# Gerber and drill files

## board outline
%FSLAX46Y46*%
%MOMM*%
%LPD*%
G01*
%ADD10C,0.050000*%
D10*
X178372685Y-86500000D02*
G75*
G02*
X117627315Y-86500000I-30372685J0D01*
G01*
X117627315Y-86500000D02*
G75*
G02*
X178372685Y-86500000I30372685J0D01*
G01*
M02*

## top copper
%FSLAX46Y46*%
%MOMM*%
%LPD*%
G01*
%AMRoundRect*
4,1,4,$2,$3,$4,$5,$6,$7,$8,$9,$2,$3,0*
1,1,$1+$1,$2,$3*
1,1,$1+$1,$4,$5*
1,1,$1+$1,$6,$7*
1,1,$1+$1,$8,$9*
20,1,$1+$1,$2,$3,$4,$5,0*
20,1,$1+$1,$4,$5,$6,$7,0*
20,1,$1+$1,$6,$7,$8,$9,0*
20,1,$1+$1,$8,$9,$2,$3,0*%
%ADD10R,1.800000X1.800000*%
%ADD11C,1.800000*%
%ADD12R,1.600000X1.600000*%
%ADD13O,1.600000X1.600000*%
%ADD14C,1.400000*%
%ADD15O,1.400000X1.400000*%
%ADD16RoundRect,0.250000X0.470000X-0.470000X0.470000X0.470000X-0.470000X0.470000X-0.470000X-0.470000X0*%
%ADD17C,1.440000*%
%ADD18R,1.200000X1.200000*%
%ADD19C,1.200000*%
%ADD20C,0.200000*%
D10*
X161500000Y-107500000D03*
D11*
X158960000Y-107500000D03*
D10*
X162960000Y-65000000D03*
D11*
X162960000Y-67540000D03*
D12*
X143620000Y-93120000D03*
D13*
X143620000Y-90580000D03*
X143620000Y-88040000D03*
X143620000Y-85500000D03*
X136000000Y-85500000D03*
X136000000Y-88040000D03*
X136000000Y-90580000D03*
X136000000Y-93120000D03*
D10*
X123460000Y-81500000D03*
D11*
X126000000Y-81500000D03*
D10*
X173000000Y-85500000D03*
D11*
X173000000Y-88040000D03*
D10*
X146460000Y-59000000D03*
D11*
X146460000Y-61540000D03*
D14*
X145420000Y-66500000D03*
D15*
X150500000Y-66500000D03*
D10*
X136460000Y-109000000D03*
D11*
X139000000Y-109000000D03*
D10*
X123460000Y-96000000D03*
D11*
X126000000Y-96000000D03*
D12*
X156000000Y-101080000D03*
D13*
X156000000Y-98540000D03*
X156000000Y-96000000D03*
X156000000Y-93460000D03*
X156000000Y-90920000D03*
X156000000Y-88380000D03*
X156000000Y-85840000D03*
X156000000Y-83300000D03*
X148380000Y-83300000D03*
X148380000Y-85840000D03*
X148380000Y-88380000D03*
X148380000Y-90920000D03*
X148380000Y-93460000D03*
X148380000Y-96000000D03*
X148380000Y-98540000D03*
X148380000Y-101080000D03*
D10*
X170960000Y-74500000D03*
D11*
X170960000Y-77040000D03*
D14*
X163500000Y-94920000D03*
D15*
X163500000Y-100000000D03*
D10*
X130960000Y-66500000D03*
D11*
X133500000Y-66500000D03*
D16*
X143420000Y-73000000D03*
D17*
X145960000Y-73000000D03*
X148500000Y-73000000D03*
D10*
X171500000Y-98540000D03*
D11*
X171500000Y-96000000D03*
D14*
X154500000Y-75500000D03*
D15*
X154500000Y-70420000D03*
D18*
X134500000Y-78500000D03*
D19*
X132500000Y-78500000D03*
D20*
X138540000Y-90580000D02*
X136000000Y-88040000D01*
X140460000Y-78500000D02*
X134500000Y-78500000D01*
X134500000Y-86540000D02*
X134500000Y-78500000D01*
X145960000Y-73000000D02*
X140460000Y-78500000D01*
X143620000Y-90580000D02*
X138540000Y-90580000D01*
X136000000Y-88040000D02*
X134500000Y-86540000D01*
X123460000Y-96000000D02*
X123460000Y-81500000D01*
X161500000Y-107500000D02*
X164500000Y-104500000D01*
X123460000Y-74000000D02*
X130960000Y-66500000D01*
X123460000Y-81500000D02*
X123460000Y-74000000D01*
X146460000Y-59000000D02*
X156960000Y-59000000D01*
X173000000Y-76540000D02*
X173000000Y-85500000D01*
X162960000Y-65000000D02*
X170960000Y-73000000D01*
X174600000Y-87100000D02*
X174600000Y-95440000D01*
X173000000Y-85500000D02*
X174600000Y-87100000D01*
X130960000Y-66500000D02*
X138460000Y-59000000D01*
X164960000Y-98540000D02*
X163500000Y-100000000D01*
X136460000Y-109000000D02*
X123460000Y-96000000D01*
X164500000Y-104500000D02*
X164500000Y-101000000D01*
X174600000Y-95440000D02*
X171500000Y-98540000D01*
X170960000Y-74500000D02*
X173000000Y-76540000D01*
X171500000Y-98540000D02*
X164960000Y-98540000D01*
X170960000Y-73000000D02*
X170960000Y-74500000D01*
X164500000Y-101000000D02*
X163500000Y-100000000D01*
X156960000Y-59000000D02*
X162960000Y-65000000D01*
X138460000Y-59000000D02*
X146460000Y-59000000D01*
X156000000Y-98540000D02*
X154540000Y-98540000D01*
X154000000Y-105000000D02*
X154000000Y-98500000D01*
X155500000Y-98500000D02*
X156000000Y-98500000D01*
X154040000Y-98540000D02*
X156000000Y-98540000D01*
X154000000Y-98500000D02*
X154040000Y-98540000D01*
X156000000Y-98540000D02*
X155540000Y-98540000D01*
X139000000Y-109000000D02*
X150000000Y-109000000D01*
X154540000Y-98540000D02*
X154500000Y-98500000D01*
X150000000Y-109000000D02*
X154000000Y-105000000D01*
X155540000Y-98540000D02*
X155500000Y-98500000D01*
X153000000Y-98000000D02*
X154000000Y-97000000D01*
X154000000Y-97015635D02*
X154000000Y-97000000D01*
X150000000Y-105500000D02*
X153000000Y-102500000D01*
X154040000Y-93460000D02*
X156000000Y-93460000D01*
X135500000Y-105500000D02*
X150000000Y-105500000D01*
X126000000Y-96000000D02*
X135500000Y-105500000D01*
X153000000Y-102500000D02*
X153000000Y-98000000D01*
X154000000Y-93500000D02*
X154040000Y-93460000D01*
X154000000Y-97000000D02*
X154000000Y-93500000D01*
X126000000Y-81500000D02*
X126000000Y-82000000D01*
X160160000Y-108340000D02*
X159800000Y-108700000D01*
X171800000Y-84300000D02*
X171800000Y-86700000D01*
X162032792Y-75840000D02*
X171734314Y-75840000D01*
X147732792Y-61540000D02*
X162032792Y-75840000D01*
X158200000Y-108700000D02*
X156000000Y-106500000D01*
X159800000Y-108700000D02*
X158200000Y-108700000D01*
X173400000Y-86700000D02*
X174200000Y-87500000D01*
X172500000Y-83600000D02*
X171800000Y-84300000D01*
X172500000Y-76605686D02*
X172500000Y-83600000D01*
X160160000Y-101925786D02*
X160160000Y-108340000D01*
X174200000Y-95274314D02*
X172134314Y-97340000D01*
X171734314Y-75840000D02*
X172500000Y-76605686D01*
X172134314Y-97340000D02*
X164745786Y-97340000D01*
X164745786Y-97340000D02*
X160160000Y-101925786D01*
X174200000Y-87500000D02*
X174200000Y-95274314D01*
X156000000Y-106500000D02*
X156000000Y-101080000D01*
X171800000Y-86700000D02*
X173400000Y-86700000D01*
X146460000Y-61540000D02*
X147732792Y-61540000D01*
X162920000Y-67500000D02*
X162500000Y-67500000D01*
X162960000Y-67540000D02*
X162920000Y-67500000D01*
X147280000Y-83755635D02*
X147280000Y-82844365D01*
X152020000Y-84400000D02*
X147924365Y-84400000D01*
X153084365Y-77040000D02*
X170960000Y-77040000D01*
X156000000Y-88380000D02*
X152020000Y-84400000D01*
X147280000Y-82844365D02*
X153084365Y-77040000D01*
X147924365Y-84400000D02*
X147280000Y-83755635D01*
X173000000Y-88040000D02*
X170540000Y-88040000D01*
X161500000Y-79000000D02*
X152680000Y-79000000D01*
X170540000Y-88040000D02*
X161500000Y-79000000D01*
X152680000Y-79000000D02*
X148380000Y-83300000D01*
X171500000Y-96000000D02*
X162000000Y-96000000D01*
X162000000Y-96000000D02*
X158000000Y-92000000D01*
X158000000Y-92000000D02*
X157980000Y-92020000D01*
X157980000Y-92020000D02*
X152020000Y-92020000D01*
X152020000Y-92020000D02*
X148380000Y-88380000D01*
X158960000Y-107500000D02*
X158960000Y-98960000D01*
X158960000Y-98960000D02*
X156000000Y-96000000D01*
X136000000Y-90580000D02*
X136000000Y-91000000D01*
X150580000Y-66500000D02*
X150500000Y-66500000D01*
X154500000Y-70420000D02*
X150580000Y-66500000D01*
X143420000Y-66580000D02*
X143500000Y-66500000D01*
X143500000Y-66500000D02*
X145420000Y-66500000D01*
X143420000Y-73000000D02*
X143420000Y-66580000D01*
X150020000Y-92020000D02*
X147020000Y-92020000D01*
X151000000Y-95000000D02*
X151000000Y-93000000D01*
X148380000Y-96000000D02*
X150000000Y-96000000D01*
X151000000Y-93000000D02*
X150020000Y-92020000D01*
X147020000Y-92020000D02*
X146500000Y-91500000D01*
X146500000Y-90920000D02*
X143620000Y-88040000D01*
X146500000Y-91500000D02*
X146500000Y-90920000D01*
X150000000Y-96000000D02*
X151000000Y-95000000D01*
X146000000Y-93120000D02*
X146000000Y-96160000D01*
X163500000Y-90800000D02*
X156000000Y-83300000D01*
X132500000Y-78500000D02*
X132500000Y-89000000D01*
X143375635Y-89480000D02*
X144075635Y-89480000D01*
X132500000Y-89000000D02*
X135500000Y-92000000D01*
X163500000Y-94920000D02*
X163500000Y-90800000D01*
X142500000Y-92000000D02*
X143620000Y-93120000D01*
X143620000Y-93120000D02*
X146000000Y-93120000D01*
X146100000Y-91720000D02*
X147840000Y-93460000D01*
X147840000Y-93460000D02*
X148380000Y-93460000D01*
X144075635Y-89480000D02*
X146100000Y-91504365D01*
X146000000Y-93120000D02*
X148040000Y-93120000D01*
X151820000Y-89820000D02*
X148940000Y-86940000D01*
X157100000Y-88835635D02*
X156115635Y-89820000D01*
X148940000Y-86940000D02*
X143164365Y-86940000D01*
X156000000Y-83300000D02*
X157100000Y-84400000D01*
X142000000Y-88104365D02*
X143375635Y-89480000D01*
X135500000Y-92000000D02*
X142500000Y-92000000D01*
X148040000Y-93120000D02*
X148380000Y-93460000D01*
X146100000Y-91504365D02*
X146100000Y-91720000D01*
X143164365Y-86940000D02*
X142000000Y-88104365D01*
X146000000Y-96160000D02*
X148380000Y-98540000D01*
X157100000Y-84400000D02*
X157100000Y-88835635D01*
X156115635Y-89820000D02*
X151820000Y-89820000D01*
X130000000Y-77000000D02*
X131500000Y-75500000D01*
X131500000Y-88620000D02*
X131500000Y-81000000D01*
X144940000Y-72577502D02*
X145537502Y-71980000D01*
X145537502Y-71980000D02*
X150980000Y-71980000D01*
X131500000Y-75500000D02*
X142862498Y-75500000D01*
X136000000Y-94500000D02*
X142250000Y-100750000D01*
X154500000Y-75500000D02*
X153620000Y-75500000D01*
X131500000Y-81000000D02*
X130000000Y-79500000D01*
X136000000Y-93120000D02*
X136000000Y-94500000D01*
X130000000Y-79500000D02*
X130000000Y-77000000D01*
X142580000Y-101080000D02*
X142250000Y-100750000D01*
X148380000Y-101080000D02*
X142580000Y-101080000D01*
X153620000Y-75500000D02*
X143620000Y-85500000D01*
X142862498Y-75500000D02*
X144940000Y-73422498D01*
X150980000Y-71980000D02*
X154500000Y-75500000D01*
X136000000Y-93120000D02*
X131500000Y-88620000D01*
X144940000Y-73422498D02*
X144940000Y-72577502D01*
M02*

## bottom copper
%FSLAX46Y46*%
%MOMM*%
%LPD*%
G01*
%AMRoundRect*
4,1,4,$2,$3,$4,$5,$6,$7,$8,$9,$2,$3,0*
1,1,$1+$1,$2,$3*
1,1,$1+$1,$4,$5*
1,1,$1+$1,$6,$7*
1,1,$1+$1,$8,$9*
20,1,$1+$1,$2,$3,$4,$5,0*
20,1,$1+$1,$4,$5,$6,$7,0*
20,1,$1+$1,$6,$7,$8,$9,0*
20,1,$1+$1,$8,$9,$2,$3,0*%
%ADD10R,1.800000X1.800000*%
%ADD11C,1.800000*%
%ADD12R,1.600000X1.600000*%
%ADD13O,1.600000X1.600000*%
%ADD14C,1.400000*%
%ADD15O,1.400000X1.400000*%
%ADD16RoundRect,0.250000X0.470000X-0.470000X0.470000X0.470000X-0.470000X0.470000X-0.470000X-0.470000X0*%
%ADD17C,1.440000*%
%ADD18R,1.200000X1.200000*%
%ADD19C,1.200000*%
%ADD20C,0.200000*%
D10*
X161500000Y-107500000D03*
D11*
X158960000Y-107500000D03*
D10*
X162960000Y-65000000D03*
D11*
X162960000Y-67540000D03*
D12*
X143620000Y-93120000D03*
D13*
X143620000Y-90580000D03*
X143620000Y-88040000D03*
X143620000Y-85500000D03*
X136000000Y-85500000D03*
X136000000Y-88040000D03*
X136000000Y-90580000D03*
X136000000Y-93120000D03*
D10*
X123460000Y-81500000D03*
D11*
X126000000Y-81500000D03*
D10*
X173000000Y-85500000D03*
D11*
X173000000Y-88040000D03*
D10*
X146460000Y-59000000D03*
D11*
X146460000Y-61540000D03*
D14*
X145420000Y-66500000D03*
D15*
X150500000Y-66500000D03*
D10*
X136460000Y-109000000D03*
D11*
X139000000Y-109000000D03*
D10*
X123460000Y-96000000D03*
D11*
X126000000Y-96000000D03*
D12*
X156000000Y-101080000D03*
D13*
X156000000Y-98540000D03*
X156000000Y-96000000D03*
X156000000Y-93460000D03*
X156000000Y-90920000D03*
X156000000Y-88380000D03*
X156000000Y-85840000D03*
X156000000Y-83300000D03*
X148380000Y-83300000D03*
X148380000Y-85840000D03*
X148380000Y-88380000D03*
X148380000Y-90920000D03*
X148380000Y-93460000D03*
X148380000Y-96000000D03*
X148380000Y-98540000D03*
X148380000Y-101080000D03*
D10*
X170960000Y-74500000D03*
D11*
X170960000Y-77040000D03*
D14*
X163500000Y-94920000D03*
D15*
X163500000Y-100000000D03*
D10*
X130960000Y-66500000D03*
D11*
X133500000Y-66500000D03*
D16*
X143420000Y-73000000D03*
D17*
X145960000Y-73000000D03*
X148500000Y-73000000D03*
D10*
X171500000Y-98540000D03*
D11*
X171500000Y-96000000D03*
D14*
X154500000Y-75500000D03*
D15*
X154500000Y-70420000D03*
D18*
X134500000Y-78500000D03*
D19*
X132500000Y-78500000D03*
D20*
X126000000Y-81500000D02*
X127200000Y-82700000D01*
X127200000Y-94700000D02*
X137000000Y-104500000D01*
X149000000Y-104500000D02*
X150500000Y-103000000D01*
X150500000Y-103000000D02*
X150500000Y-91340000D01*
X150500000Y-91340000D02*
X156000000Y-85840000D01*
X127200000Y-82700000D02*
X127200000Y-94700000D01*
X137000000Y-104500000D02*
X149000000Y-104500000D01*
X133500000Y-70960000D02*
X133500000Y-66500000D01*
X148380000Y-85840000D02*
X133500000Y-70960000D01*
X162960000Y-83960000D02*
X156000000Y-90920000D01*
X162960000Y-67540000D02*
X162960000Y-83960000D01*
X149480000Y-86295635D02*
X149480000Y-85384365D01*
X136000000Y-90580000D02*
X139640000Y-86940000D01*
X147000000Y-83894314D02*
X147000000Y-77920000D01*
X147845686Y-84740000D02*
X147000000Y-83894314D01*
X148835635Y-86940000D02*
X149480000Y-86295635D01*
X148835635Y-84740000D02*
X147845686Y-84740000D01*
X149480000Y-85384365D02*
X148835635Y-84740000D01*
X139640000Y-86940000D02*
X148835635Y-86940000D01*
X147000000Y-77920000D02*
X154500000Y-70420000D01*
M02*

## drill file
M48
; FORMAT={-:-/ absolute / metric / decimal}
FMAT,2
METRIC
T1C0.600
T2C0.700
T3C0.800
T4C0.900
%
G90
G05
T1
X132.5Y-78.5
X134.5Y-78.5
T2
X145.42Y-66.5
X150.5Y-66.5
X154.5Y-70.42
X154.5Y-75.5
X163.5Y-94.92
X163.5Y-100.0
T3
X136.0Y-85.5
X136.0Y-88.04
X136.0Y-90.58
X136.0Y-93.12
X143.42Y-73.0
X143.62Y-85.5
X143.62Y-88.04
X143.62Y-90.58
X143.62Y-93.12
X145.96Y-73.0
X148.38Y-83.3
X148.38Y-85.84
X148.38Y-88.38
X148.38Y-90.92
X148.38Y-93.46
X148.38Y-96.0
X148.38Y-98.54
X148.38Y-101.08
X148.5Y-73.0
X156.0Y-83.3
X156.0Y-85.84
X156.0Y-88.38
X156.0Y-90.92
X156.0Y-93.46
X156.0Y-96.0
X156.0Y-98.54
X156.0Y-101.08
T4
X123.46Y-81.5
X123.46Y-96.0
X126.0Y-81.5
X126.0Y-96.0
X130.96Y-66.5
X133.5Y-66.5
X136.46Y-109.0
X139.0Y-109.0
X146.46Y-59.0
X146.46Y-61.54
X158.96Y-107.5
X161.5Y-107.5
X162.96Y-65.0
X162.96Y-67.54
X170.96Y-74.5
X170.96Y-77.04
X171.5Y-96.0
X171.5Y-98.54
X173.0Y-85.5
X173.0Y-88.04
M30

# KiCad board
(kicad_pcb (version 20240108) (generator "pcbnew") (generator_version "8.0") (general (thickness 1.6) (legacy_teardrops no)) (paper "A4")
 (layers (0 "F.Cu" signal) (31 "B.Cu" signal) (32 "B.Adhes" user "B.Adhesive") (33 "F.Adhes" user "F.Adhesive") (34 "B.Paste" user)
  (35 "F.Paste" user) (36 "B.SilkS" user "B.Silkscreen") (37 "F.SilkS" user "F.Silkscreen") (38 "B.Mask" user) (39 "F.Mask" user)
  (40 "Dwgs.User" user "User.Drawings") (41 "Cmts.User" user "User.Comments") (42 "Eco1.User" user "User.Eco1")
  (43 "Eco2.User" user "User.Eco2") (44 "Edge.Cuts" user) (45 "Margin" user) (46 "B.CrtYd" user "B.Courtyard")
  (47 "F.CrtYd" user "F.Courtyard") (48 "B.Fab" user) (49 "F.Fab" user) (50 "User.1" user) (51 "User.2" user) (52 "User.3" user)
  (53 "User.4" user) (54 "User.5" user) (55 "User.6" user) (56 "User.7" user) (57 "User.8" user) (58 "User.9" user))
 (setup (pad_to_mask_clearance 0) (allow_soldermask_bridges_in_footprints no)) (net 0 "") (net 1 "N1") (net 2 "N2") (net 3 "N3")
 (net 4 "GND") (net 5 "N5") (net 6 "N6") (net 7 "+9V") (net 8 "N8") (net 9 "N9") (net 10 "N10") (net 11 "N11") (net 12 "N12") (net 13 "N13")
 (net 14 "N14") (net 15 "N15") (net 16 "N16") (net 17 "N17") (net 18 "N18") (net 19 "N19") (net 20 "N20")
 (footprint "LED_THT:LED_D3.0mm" (layer "F.Cu") (at 161.5 107.5 180)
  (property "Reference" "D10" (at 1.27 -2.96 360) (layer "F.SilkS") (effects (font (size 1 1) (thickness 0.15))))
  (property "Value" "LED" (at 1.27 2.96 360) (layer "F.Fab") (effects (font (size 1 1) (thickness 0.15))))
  (pad "1" thru_hole rect (at 0 0 180) (size 1.8 1.8) (drill 0.9) (layers "*.Cu" "*.Mask") (remove_unused_layers no) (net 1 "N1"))
  (pad "2" thru_hole circle (at 2.54 0 180) (size 1.8 1.8) (drill 0.9) (layers "*.Cu" "*.Mask") (remove_unused_layers no) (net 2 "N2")))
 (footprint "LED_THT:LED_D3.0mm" (layer "F.Cu") (at 162.96 65 -90)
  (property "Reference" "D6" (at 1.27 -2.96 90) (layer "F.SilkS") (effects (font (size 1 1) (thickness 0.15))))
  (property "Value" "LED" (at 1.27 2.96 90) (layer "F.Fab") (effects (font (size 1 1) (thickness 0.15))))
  (pad "1" thru_hole rect (at 0 0 270) (size 1.8 1.8) (drill 0.9) (layers "*.Cu" "*.Mask") (remove_unused_layers no) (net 1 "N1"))
  (pad "2" thru_hole circle (at 2.54 0 270) (size 1.8 1.8) (drill 0.9) (layers "*.Cu" "*.Mask") (remove_unused_layers no) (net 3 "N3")))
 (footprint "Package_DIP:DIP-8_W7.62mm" (layer "F.Cu") (at 143.62 93.12 180)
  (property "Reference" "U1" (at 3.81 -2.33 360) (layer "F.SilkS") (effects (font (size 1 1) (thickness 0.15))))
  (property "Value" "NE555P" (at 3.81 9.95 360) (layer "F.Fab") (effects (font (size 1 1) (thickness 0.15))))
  (pad "1" thru_hole rect (at 0 0 180) (size 1.6 1.6) (drill 0.8) (layers "*.Cu" "*.Mask") (remove_unused_layers no) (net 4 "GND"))
  (pad "2" thru_hole oval (at 0 2.54 180) (size 1.6 1.6) (drill 0.8) (layers "*.Cu" "*.Mask") (remove_unused_layers no) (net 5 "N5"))
  (pad "3" thru_hole oval (at 0 5.08 180) (size 1.6 1.6) (drill 0.8) (layers "*.Cu" "*.Mask") (remove_unused_layers no) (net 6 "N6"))
  (pad "4" thru_hole oval (at 0 7.62 180) (size 1.6 1.6) (drill 0.8) (layers "*.Cu" "*.Mask") (remove_unused_layers no) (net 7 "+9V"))
  (pad "5" thru_hole oval (at 7.62 7.62 180) (size 1.6 1.6) (drill 0.8) (layers "*.Cu" "*.Mask") (remove_unused_layers no) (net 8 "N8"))
  (pad "6" thru_hole oval (at 7.62 5.08 180) (size 1.6 1.6) (drill 0.8) (layers "*.Cu" "*.Mask") (remove_unused_layers no) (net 5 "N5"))
  (pad "7" thru_hole oval (at 7.62 2.54 180) (size 1.6 1.6) (drill 0.8) (layers "*.Cu" "*.Mask") (remove_unused_layers no) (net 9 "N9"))
  (pad "8" thru_hole oval (at 7.62 0 180) (size 1.6 1.6) (drill 0.8) (layers "*.Cu" "*.Mask") (remove_unused_layers no) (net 7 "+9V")))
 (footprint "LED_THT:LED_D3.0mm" (layer "F.Cu") (at 123.46 81.5)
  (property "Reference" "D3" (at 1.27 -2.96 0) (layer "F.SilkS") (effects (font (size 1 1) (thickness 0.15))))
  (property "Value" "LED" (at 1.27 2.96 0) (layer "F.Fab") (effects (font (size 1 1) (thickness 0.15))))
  (pad "1" thru_hole rect (at 0 0) (size 1.8 1.8) (drill 0.9) (layers "*.Cu" "*.Mask") (remove_unused_layers no) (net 1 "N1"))
  (pad "2" thru_hole circle (at 2.54 0) (size 1.8 1.8) (drill 0.9) (layers "*.Cu" "*.Mask") (remove_unused_layers no) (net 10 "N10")))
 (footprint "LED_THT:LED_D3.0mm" (layer "F.Cu") (at 173 85.5 -90)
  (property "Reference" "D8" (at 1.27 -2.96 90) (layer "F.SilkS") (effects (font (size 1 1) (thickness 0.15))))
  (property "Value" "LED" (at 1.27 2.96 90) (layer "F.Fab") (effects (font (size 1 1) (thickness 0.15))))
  (pad "1" thru_hole rect (at 0 0 270) (size 1.8 1.8) (drill 0.9) (layers "*.Cu" "*.Mask") (remove_unused_layers no) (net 1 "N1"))
  (pad "2" thru_hole circle (at 2.54 0 270) (size 1.8 1.8) (drill 0.9) (layers "*.Cu" "*.Mask") (remove_unused_layers no) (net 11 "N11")))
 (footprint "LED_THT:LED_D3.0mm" (layer "F.Cu") (at 146.46 59 -90)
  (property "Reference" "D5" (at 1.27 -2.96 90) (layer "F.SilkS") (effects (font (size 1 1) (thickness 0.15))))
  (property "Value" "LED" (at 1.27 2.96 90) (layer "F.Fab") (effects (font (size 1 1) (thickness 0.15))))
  (pad "1" thru_hole rect (at 0 0 270) (size 1.8 1.8) (drill 0.9) (layers "*.Cu" "*.Mask") (remove_unused_layers no) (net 1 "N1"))
  (pad "2" thru_hole circle (at 2.54 0 270) (size 1.8 1.8) (drill 0.9) (layers "*.Cu" "*.Mask") (remove_unused_layers no) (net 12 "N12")))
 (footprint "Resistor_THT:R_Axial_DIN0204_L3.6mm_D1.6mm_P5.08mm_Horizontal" (layer "F.Cu") (at 145.42 66.5)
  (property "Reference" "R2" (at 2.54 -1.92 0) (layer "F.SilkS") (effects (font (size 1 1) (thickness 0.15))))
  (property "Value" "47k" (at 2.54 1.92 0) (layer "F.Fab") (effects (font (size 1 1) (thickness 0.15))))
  (pad "1" thru_hole circle (at 0 0) (size 1.4 1.4) (drill 0.7) (layers "*.Cu" "*.Mask") (remove_unused_layers no) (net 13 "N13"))
  (pad "2" thru_hole oval (at 5.08 0) (size 1.4 1.4) (drill 0.7) (layers "*.Cu" "*.Mask") (remove_unused_layers no) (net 9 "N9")))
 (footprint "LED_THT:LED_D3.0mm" (layer "F.Cu") (at 136.46 109)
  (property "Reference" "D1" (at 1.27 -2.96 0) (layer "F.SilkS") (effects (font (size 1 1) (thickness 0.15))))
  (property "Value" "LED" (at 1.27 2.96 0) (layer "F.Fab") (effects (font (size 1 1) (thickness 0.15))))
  (pad "1" thru_hole rect (at 0 0) (size 1.8 1.8) (drill 0.9) (layers "*.Cu" "*.Mask") (remove_unused_layers no) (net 1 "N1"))
  (pad "2" thru_hole circle (at 2.54 0) (size 1.8 1.8) (drill 0.9) (layers "*.Cu" "*.Mask") (remove_unused_layers no) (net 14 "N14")))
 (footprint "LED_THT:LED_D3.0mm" (layer "F.Cu") (at 123.46 96)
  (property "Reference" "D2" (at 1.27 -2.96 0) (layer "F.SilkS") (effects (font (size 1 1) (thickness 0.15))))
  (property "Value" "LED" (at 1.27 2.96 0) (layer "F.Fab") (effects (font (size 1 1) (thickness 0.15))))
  (pad "1" thru_hole rect (at 0 0) (size 1.8 1.8) (drill 0.9) (layers "*.Cu" "*.Mask") (remove_unused_layers no) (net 1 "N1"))
  (pad "2" thru_hole circle (at 2.54 0) (size 1.8 1.8) (drill 0.9) (layers "*.Cu" "*.Mask") (remove_unused_layers no) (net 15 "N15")))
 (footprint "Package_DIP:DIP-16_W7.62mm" (layer "F.Cu") (at 156 101.08 180)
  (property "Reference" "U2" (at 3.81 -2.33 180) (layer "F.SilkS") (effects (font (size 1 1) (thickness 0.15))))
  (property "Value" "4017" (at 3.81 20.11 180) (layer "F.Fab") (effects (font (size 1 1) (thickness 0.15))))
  (pad "1" thru_hole rect (at 0 0 180) (size 1.6 1.6) (drill 0.8) (layers "*.Cu" "*.Mask") (remove_unused_layers no) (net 12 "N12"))
  (pad "2" thru_hole oval (at 0 2.54 180) (size 1.6 1.6) (drill 0.8) (layers "*.Cu" "*.Mask") (remove_unused_layers no) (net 14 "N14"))
  (pad "3" thru_hole oval (at 0 5.08 180) (size 1.6 1.6) (drill 0.8) (layers "*.Cu" "*.Mask") (remove_unused_layers no) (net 2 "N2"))
  (pad "4" thru_hole oval (at 0 7.62 180) (size 1.6 1.6) (drill 0.8) (layers "*.Cu" "*.Mask") (remove_unused_layers no) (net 15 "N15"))
  (pad "5" thru_hole oval (at 0 10.16 180) (size 1.6 1.6) (drill 0.8) (layers "*.Cu" "*.Mask") (remove_unused_layers no) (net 3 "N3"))
  (pad "6" thru_hole oval (at 0 12.7 180) (size 1.6 1.6) (drill 0.8) (layers "*.Cu" "*.Mask") (remove_unused_layers no) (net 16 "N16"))
  (pad "7" thru_hole oval (at 0 15.24 180) (size 1.6 1.6) (drill 0.8) (layers "*.Cu" "*.Mask") (remove_unused_layers no) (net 10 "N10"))
  (pad "8" thru_hole oval (at 0 17.78 180) (size 1.6 1.6) (drill 0.8) (layers "*.Cu" "*.Mask") (remove_unused_layers no) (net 4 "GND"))
  (pad "9" thru_hole oval (at 7.62 17.78 180) (size 1.6 1.6) (drill 0.8) (layers "*.Cu" "*.Mask") (remove_unused_layers no) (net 11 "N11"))
  (pad "10" thru_hole oval (at 7.62 15.24 180) (size 1.6 1.6) (drill 0.8) (layers "*.Cu" "*.Mask") (remove_unused_layers no) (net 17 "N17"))
  (pad "11" thru_hole oval (at 7.62 12.7 180) (size 1.6 1.6) (drill 0.8) (layers "*.Cu" "*.Mask") (remove_unused_layers no) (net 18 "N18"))
  (pad "12" thru_hole oval (at 7.62 10.16 180) (size 1.6 1.6) (drill 0.8) (layers "*.Cu" "*.Mask") (remove_unused_layers no) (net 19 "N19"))
  (pad "13" thru_hole oval (at 7.62 7.62 180) (size 1.6 1.6) (drill 0.8) (layers "*.Cu" "*.Mask") (remove_unused_layers no) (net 4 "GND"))
  (pad "14" thru_hole oval (at 7.62 5.08 180) (size 1.6 1.6) (drill 0.8) (layers "*.Cu" "*.Mask") (remove_unused_layers no) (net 6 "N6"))
  (pad "15" thru_hole oval (at 7.62 2.54 180) (size 1.6 1.6) (drill 0.8) (layers "*.Cu" "*.Mask") (remove_unused_layers no) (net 4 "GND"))
  (pad "16" thru_hole oval (at 7.62 0 180) (size 1.6 1.6) (drill 0.8) (layers "*.Cu" "*.Mask") (remove_unused_layers no) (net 7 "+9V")))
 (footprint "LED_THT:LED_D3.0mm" (layer "F.Cu") (at 170.96 74.5 -90)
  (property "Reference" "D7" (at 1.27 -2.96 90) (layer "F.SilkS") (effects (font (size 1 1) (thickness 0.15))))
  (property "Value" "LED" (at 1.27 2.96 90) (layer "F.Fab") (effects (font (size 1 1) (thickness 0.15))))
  (pad "1" thru_hole rect (at 0 0 270) (size 1.8 1.8) (drill 0.9) (layers "*.Cu" "*.Mask") (remove_unused_layers no) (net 1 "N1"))
  (pad "2" thru_hole circle (at 2.54 0 270) (size 1.8 1.8) (drill 0.9) (layers "*.Cu" "*.Mask") (remove_unused_layers no) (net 16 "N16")))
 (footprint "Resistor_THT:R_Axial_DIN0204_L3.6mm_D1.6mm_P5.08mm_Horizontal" (layer "F.Cu") (at 163.5 94.92 -90)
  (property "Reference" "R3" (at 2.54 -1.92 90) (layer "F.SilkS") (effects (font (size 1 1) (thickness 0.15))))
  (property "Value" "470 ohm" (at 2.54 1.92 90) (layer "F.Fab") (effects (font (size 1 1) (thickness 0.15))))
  (pad "1" thru_hole circle (at 0 0 270) (size 1.4 1.4) (drill 0.7) (layers "*.Cu" "*.Mask") (remove_unused_layers no) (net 4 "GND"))
  (pad "2" thru_hole oval (at 5.08 0 270) (size 1.4 1.4) (drill 0.7) (layers "*.Cu" "*.Mask") (remove_unused_layers no) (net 1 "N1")))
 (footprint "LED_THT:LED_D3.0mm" (layer "F.Cu") (at 130.96 66.5)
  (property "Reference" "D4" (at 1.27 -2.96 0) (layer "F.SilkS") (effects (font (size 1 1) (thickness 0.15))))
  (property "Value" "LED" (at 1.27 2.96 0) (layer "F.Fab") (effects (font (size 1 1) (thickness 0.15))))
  (pad "1" thru_hole rect (at 0 0) (size 1.8 1.8) (drill 0.9) (layers "*.Cu" "*.Mask") (remove_unused_layers no) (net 1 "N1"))
  (pad "2" thru_hole circle (at 2.54 0) (size 1.8 1.8) (drill 0.9) (layers "*.Cu" "*.Mask") (remove_unused_layers no) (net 17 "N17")))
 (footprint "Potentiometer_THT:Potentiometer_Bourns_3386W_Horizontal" (layer "F.Cu") (at 143.42 73)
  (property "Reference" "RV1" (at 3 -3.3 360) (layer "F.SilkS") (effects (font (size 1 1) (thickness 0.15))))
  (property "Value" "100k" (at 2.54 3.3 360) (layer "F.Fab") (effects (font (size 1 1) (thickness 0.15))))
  (pad "1" thru_hole roundrect (at 0 0 90) (size 1.44 1.44) (drill 0.8) (layers "*.Cu" "*.Mask") (remove_unused_layers no)
   (roundrect_rratio 0.1736111111) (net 13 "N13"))
  (pad "2" thru_hole circle (at 2.54 0 90) (size 1.44 1.44) (drill 0.8) (layers "*.Cu" "*.Mask") (remove_unused_layers no) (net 5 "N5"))
  (pad "3" thru_hole circle (at 5.08 0 90) (size 1.44 1.44) (drill 0.8) (layers "*.Cu" "*.Mask") (remove_unused_layers no) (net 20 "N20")))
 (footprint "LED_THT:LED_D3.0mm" (layer "F.Cu") (at 171.5 98.54 90)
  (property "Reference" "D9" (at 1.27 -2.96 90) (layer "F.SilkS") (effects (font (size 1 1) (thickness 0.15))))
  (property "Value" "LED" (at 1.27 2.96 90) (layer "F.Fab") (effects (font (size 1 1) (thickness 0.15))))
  (pad "1" thru_hole rect (at 0 0 90) (size 1.8 1.8) (drill 0.9) (layers "*.Cu" "*.Mask") (remove_unused_layers no) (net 1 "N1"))
  (pad "2" thru_hole circle (at 2.54 0 90) (size 1.8 1.8) (drill 0.9) (layers "*.Cu" "*.Mask") (remove_unused_layers no) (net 18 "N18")))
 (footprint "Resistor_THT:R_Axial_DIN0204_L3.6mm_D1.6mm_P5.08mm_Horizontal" (layer "F.Cu") (at 154.5 75.5 90)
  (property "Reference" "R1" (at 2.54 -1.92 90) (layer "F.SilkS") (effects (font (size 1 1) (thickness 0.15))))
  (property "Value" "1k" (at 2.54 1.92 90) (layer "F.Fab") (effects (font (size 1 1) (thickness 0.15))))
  (pad "1" thru_hole circle (at 0 0 90) (size 1.4 1.4) (drill 0.7) (layers "*.Cu" "*.Mask") (remove_unused_layers no) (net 7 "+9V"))
  (pad "2" thru_hole oval (at 5.08 0 90) (size 1.4 1.4) (drill 0.7) (layers "*.Cu" "*.Mask") (remove_unused_layers no) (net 9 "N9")))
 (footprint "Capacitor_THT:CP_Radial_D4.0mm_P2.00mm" (layer "F.Cu") (at 134.5 78.5 180)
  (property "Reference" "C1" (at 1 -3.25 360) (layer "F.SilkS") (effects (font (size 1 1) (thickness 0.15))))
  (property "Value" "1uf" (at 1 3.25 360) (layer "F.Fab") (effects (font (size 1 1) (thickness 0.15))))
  (pad "1" thru_hole rect (at 0 0 180) (size 1.2 1.2) (drill 0.6) (layers "*.Cu" "*.Mask") (remove_unused_layers no) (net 5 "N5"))
  (pad "2" thru_hole circle (at 2 0 180) (size 1.2 1.2) (drill 0.6) (layers "*.Cu" "*.Mask") (remove_unused_layers no) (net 4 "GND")))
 (gr_circle (center 148 86.5) (end 173.5 103) (stroke (width 0.05) (type default)) (fill none) (layer "Edge.Cuts"))
 (segment (start 138.54 90.58) (end 136 88.04) (width 0.2) (layer "F.Cu") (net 5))
 (segment (start 140.46 78.5) (end 134.5 78.5) (width 0.2) (layer "F.Cu") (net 5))
 (segment (start 134.5 86.54) (end 134.5 78.5) (width 0.2) (layer "F.Cu") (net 5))
 (segment (start 145.96 73) (end 140.46 78.5) (width 0.2) (layer "F.Cu") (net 5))
 (segment (start 143.62 90.58) (end 138.54 90.58) (width 0.2) (layer "F.Cu") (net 5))
 (segment (start 136 88.04) (end 134.5 86.54) (width 0.2) (layer "F.Cu") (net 5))
 (segment (start 123.46 96) (end 123.46 81.5) (width 0.2) (layer "F.Cu") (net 1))
 (segment (start 161.5 107.5) (end 164.5 104.5) (width 0.2) (layer "F.Cu") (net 1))
 (segment (start 123.46 74) (end 130.96 66.5) (width 0.2) (layer "F.Cu") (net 1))
 (segment (start 123.46 81.5) (end 123.46 74) (width 0.2) (layer "F.Cu") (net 1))
 (segment (start 146.46 59) (end 156.96 59) (width 0.2) (layer "F.Cu") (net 1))
 (segment (start 173 76.54) (end 173 85.5) (width 0.2) (layer "F.Cu") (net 1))
 (segment (start 162.96 65) (end 170.96 73) (width 0.2) (layer "F.Cu") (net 1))
 (segment (start 174.6 87.1) (end 174.6 95.44) (width 0.2) (layer "F.Cu") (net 1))
 (segment (start 173 85.5) (end 174.6 87.1) (width 0.2) (layer "F.Cu") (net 1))
 (segment (start 130.96 66.5) (end 138.46 59) (width 0.2) (layer "F.Cu") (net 1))
 (segment (start 164.96 98.54) (end 163.5 100) (width 0.2) (layer "F.Cu") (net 1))
 (segment (start 136.46 109) (end 123.46 96) (width 0.2) (layer "F.Cu") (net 1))
 (segment (start 164.5 104.5) (end 164.5 101) (width 0.2) (layer "F.Cu") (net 1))
 (segment (start 174.6 95.44) (end 171.5 98.54) (width 0.2) (layer "F.Cu") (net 1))
 (segment (start 170.96 74.5) (end 173 76.54) (width 0.2) (layer "F.Cu") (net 1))
 (segment (start 171.5 98.54) (end 164.96 98.54) (width 0.2) (layer "F.Cu") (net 1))
 (segment (start 170.96 73) (end 170.96 74.5) (width 0.2) (layer "F.Cu") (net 1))
 (segment (start 164.5 101) (end 163.5 100) (width 0.2) (layer "F.Cu") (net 1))
 (segment (start 156.96 59) (end 162.96 65) (width 0.2) (layer "F.Cu") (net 1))
 (segment (start 138.46 59) (end 146.46 59) (width 0.2) (layer "F.Cu") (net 1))
 (segment (start 156 98.54) (end 154.54 98.54) (width 0.2) (layer "F.Cu") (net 14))
 (segment (start 154 105) (end 154 98.5) (width 0.2) (layer "F.Cu") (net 14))
 (segment (start 155.5 98.5) (end 156 98.5) (width 0.2) (layer "F.Cu") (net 14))
 (segment (start 154.04 98.54) (end 156 98.54) (width 0.2) (layer "F.Cu") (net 14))
 (segment (start 154 98.5) (end 154.04 98.54) (width 0.2) (layer "F.Cu") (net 14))
 (segment (start 156 98.54) (end 155.54 98.54) (width 0.2) (layer "F.Cu") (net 14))
 (segment (start 139 109) (end 150 109) (width 0.2) (layer "F.Cu") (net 14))
 (segment (start 154.54 98.54) (end 154.5 98.5) (width 0.2) (layer "F.Cu") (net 14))
 (segment (start 150 109) (end 154 105) (width 0.2) (layer "F.Cu") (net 14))
 (segment (start 155.54 98.54) (end 155.5 98.5) (width 0.2) (layer "F.Cu") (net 14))
 (segment (start 153 98) (end 154 97) (width 0.2) (layer "F.Cu") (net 15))
 (segment (start 154 97.015635) (end 154 97) (width 0.2) (layer "F.Cu") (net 15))
 (segment (start 150 105.5) (end 153 102.5) (width 0.2) (layer "F.Cu") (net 15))
 (segment (start 154.04 93.46) (end 156 93.46) (width 0.2) (layer "F.Cu") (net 15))
 (segment (start 135.5 105.5) (end 150 105.5) (width 0.2) (layer "F.Cu") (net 15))
 (segment (start 126 96) (end 135.5 105.5) (width 0.2) (layer "F.Cu") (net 15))
 (segment (start 153 102.5) (end 153 98) (width 0.2) (layer "F.Cu") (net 15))
 (segment (start 154 93.5) (end 154.04 93.46) (width 0.2) (layer "F.Cu") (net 15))
 (segment (start 154 97) (end 154 93.5) (width 0.2) (layer "F.Cu") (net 15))
 (segment (start 126 81.5) (end 126 82) (width 0.2) (layer "F.Cu") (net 10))
 (segment (start 126 81.5) (end 127.2 82.7) (width 0.2) (layer "B.Cu") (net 10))
 (segment (start 127.2 94.7) (end 137 104.5) (width 0.2) (layer "B.Cu") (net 10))
 (segment (start 149 104.5) (end 150.5 103) (width 0.2) (layer "B.Cu") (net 10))
 (segment (start 150.5 103) (end 150.5 91.34) (width 0.2) (layer "B.Cu") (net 10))
 (segment (start 150.5 91.34) (end 156 85.84) (width 0.2) (layer "B.Cu") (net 10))
 (segment (start 127.2 82.7) (end 127.2 94.7) (width 0.2) (layer "B.Cu") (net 10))
 (segment (start 137 104.5) (end 149 104.5) (width 0.2) (layer "B.Cu") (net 10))
 (segment (start 133.5 70.96) (end 133.5 66.5) (width 0.2) (layer "B.Cu") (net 17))
 (segment (start 148.38 85.84) (end 133.5 70.96) (width 0.2) (layer "B.Cu") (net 17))
 (segment (start 160.16 108.34) (end 159.8 108.7) (width 0.2) (layer "F.Cu") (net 12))
 (segment (start 171.8 84.3) (end 171.8 86.7) (width 0.2) (layer "F.Cu") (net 12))
 (segment (start 162.032792 75.84) (end 171.734314 75.84) (width 0.2) (layer "F.Cu") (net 12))
 (segment (start 147.732792 61.54) (end 162.032792 75.84) (width 0.2) (layer "F.Cu") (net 12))
 (segment (start 158.2 108.7) (end 156 106.5) (width 0.2) (layer "F.Cu") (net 12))
 (segment (start 159.8 108.7) (end 158.2 108.7) (width 0.2) (layer "F.Cu") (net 12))
 (segment (start 173.4 86.7) (end 174.2 87.5) (width 0.2) (layer "F.Cu") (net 12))
 (segment (start 172.5 83.6) (end 171.8 84.3) (width 0.2) (layer "F.Cu") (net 12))
 (segment (start 172.5 76.605686) (end 172.5 83.6) (width 0.2) (layer "F.Cu") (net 12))
 (segment (start 160.16 101.925786) (end 160.16 108.34) (width 0.2) (layer "F.Cu") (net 12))
 (segment (start 174.2 95.274314) (end 172.134314 97.34) (width 0.2) (layer "F.Cu") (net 12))
 (segment (start 171.734314 75.84) (end 172.5 76.605686) (width 0.2) (layer "F.Cu") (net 12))
 (segment (start 172.134314 97.34) (end 164.745786 97.34) (width 0.2) (layer "F.Cu") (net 12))
 (segment (start 164.745786 97.34) (end 160.16 101.925786) (width 0.2) (layer "F.Cu") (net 12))
 (segment (start 174.2 87.5) (end 174.2 95.274314) (width 0.2) (layer "F.Cu") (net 12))
 (segment (start 156 106.5) (end 156 101.08) (width 0.2) (layer "F.Cu") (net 12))
 (segment (start 171.8 86.7) (end 173.4 86.7) (width 0.2) (layer "F.Cu") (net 12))
 (segment (start 146.46 61.54) (end 147.732792 61.54) (width 0.2) (layer "F.Cu") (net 12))
 (segment (start 162.92 67.5) (end 162.5 67.5) (width 0.2) (layer "F.Cu") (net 3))
 (segment (start 162.96 67.54) (end 162.92 67.5) (width 0.2) (layer "F.Cu") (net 3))
 (segment (start 162.96 83.96) (end 156 90.92) (width 0.2) (layer "B.Cu") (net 3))
 (segment (start 162.96 67.54) (end 162.96 83.96) (width 0.2) (layer "B.Cu") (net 3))
 (segment (start 147.28 83.755635) (end 147.28 82.844365) (width 0.2) (layer "F.Cu") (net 16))
 (segment (start 152.02 84.4) (end 147.924365 84.4) (width 0.2) (layer "F.Cu") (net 16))
 (segment (start 153.084365 77.04) (end 170.96 77.04) (width 0.2) (layer "F.Cu") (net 16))
 (segment (start 156 88.38) (end 152.02 84.4) (width 0.2) (layer "F.Cu") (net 16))
 (segment (start 147.28 82.844365) (end 153.084365 77.04) (width 0.2) (layer "F.Cu") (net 16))
 (segment (start 147.924365 84.4) (end 147.28 83.755635) (width 0.2) (layer "F.Cu") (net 16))
 (segment (start 173 88.04) (end 170.54 88.04) (width 0.2) (layer "F.Cu") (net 11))
 (segment (start 161.5 79) (end 152.68 79) (width 0.2) (layer "F.Cu") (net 11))
 (segment (start 170.54 88.04) (end 161.5 79) (width 0.2) (layer "F.Cu") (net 11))
 (segment (start 152.68 79) (end 148.38 83.3) (width 0.2) (layer "F.Cu") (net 11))
 (segment (start 171.5 96) (end 162 96) (width 0.2) (layer "F.Cu") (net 18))
 (segment (start 162 96) (end 158 92) (width 0.2) (layer "F.Cu") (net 18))
 (segment (start 158 92) (end 157.98 92.02) (width 0.2) (layer "F.Cu") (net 18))
 (segment (start 157.98 92.02) (end 152.02 92.02) (width 0.2) (layer "F.Cu") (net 18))
 (segment (start 152.02 92.02) (end 148.38 88.38) (width 0.2) (layer "F.Cu") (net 18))
 (segment (start 158.96 107.5) (end 158.96 98.96) (width 0.2) (layer "F.Cu") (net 2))
 (segment (start 158.96 98.96) (end 156 96) (width 0.2) (layer "F.Cu") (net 2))
 (segment (start 136 90.58) (end 136 91) (width 0.2) (layer "F.Cu") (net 9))
 (segment (start 150.58 66.5) (end 150.5 66.5) (width 0.2) (layer "F.Cu") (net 9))
 (segment (start 154.5 70.42) (end 150.58 66.5) (width 0.2) (layer "F.Cu") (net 9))
 (segment (start 149.48 86.295635) (end 149.48 85.384365) (width 0.2) (layer "B.Cu") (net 9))
 (segment (start 136 90.58) (end 139.64 86.94) (width 0.2) (layer "B.Cu") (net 9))
 (segment (start 147 83.894314) (end 147 77.92) (width 0.2) (layer "B.Cu") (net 9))
 (segment (start 147.845686 84.74) (end 147 83.894314) (width 0.2) (layer "B.Cu") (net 9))
 (segment (start 148.835635 86.94) (end 149.48 86.295635) (width 0.2) (layer "B.Cu") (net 9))
 (segment (start 148.835635 84.74) (end 147.845686 84.74) (width 0.2) (layer "B.Cu") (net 9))
 (segment (start 149.48 85.384365) (end 148.835635 84.74) (width 0.2) (layer "B.Cu") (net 9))
 (segment (start 139.64 86.94) (end 148.835635 86.94) (width 0.2) (layer "B.Cu") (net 9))
 (segment (start 147 77.92) (end 154.5 70.42) (width 0.2) (layer "B.Cu") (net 9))
 (segment (start 143.42 66.58) (end 143.5 66.5) (width 0.2) (layer "F.Cu") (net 13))
 (segment (start 143.5 66.5) (end 145.42 66.5) (width 0.2) (layer "F.Cu") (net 13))
 (segment (start 143.42 73) (end 143.42 66.58) (width 0.2) (layer "F.Cu") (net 13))
 (segment (start 150.02 92.02) (end 147.02 92.02) (width 0.2) (layer "F.Cu") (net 6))
 (segment (start 151 95) (end 151 93) (width 0.2) (layer "F.Cu") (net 6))
 (segment (start 148.38 96) (end 150 96) (width 0.2) (layer "F.Cu") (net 6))
 (segment (start 151 93) (end 150.02 92.02) (width 0.2) (layer "F.Cu") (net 6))
 (segment (start 147.02 92.02) (end 146.5 91.5) (width 0.2) (layer "F.Cu") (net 6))
 (segment (start 146.5 90.92) (end 143.62 88.04) (width 0.2) (layer "F.Cu") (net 6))
 (segment (start 146.5 91.5) (end 146.5 90.92) (width 0.2) (layer "F.Cu") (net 6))
 (segment (start 150 96) (end 151 95) (width 0.2) (layer "F.Cu") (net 6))
 (segment (start 146 93.12) (end 146 96.16) (width 0.2) (layer "F.Cu") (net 4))
 (segment (start 163.5 90.8) (end 156 83.3) (width 0.2) (layer "F.Cu") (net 4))
 (segment (start 132.5 78.5) (end 132.5 89) (width 0.2) (layer "F.Cu") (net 4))
 (segment (start 143.375635 89.48) (end 144.075635 89.48) (width 0.2) (layer "F.Cu") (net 4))
 (segment (start 132.5 89) (end 135.5 92) (width 0.2) (layer "F.Cu") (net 4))
 (segment (start 163.5 94.92) (end 163.5 90.8) (width 0.2) (layer "F.Cu") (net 4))
 (segment (start 142.5 92) (end 143.62 93.12) (width 0.2) (layer "F.Cu") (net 4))
 (segment (start 143.62 93.12) (end 146 93.12) (width 0.2) (layer "F.Cu") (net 4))
 (segment (start 146.1 91.72) (end 147.84 93.46) (width 0.2) (layer "F.Cu") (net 4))
 (segment (start 147.84 93.46) (end 148.38 93.46) (width 0.2) (layer "F.Cu") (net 4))
 (segment (start 144.075635 89.48) (end 146.1 91.504365) (width 0.2) (layer "F.Cu") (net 4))
 (segment (start 146 93.12) (end 148.04 93.12) (width 0.2) (layer "F.Cu") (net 4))
 (segment (start 151.82 89.82) (end 148.94 86.94) (width 0.2) (layer "F.Cu") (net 4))
 (segment (start 157.1 88.835635) (end 156.115635 89.82) (width 0.2) (layer "F.Cu") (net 4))
 (segment (start 148.94 86.94) (end 143.164365 86.94) (width 0.2) (layer "F.Cu") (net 4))
 (segment (start 156 83.3) (end 157.1 84.4) (width 0.2) (layer "F.Cu") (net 4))
 (segment (start 142 88.104365) (end 143.375635 89.48) (width 0.2) (layer "F.Cu") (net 4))
 (segment (start 135.5 92) (end 142.5 92) (width 0.2) (layer "F.Cu") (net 4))
 (segment (start 148.04 93.12) (end 148.38 93.46) (width 0.2) (layer "F.Cu") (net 4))
 (segment (start 146.1 91.504365) (end 146.1 91.72) (width 0.2) (layer "F.Cu") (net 4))
 (segment (start 143.164365 86.94) (end 142 88.104365) (width 0.2) (layer "F.Cu") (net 4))
 (segment (start 146 96.16) (end 148.38 98.54) (width 0.2) (layer "F.Cu") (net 4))
 (segment (start 157.1 84.4) (end 157.1 88.835635) (width 0.2) (layer "F.Cu") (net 4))
 (segment (start 156.115635 89.82) (end 151.82 89.82) (width 0.2) (layer "F.Cu") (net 4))
 (segment (start 130 77) (end 131.5 75.5) (width 0.2) (layer "F.Cu") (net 7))
 (segment (start 131.5 88.62) (end 131.5 81) (width 0.2) (layer "F.Cu") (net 7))
 (segment (start 144.94 72.577502) (end 145.537502 71.98) (width 0.2) (layer "F.Cu") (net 7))
 (segment (start 145.537502 71.98) (end 150.98 71.98) (width 0.2) (layer "F.Cu") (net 7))
 (segment (start 131.5 75.5) (end 142.862498 75.5) (width 0.2) (layer "F.Cu") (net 7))
 (segment (start 136 94.5) (end 142.25 100.75) (width 0.2) (layer "F.Cu") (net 7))
 (segment (start 154.5 75.5) (end 153.62 75.5) (width 0.2) (layer "F.Cu") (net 7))
 (segment (start 131.5 81) (end 130 79.5) (width 0.2) (layer "F.Cu") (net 7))
 (segment (start 136 93.12) (end 136 94.5) (width 0.2) (layer "F.Cu") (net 7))
 (segment (start 130 79.5) (end 130 77) (width 0.2) (layer "F.Cu") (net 7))
 (segment (start 142.58 101.08) (end 142.25 100.75) (width 0.2) (layer "F.Cu") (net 7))
 (segment (start 148.38 101.08) (end 142.58 101.08) (width 0.2) (layer "F.Cu") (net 7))
 (segment (start 153.62 75.5) (end 143.62 85.5) (width 0.2) (layer "F.Cu") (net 7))
 (segment (start 142.862498 75.5) (end 144.94 73.422498) (width 0.2) (layer "F.Cu") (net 7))
 (segment (start 150.98 71.98) (end 154.5 75.5) (width 0.2) (layer "F.Cu") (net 7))
 (segment (start 136 93.12) (end 131.5 88.62) (width 0.2) (layer "F.Cu") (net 7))
 (segment (start 144.94 73.422498) (end 144.94 72.577502) (width 0.2) (layer "F.Cu") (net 7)))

